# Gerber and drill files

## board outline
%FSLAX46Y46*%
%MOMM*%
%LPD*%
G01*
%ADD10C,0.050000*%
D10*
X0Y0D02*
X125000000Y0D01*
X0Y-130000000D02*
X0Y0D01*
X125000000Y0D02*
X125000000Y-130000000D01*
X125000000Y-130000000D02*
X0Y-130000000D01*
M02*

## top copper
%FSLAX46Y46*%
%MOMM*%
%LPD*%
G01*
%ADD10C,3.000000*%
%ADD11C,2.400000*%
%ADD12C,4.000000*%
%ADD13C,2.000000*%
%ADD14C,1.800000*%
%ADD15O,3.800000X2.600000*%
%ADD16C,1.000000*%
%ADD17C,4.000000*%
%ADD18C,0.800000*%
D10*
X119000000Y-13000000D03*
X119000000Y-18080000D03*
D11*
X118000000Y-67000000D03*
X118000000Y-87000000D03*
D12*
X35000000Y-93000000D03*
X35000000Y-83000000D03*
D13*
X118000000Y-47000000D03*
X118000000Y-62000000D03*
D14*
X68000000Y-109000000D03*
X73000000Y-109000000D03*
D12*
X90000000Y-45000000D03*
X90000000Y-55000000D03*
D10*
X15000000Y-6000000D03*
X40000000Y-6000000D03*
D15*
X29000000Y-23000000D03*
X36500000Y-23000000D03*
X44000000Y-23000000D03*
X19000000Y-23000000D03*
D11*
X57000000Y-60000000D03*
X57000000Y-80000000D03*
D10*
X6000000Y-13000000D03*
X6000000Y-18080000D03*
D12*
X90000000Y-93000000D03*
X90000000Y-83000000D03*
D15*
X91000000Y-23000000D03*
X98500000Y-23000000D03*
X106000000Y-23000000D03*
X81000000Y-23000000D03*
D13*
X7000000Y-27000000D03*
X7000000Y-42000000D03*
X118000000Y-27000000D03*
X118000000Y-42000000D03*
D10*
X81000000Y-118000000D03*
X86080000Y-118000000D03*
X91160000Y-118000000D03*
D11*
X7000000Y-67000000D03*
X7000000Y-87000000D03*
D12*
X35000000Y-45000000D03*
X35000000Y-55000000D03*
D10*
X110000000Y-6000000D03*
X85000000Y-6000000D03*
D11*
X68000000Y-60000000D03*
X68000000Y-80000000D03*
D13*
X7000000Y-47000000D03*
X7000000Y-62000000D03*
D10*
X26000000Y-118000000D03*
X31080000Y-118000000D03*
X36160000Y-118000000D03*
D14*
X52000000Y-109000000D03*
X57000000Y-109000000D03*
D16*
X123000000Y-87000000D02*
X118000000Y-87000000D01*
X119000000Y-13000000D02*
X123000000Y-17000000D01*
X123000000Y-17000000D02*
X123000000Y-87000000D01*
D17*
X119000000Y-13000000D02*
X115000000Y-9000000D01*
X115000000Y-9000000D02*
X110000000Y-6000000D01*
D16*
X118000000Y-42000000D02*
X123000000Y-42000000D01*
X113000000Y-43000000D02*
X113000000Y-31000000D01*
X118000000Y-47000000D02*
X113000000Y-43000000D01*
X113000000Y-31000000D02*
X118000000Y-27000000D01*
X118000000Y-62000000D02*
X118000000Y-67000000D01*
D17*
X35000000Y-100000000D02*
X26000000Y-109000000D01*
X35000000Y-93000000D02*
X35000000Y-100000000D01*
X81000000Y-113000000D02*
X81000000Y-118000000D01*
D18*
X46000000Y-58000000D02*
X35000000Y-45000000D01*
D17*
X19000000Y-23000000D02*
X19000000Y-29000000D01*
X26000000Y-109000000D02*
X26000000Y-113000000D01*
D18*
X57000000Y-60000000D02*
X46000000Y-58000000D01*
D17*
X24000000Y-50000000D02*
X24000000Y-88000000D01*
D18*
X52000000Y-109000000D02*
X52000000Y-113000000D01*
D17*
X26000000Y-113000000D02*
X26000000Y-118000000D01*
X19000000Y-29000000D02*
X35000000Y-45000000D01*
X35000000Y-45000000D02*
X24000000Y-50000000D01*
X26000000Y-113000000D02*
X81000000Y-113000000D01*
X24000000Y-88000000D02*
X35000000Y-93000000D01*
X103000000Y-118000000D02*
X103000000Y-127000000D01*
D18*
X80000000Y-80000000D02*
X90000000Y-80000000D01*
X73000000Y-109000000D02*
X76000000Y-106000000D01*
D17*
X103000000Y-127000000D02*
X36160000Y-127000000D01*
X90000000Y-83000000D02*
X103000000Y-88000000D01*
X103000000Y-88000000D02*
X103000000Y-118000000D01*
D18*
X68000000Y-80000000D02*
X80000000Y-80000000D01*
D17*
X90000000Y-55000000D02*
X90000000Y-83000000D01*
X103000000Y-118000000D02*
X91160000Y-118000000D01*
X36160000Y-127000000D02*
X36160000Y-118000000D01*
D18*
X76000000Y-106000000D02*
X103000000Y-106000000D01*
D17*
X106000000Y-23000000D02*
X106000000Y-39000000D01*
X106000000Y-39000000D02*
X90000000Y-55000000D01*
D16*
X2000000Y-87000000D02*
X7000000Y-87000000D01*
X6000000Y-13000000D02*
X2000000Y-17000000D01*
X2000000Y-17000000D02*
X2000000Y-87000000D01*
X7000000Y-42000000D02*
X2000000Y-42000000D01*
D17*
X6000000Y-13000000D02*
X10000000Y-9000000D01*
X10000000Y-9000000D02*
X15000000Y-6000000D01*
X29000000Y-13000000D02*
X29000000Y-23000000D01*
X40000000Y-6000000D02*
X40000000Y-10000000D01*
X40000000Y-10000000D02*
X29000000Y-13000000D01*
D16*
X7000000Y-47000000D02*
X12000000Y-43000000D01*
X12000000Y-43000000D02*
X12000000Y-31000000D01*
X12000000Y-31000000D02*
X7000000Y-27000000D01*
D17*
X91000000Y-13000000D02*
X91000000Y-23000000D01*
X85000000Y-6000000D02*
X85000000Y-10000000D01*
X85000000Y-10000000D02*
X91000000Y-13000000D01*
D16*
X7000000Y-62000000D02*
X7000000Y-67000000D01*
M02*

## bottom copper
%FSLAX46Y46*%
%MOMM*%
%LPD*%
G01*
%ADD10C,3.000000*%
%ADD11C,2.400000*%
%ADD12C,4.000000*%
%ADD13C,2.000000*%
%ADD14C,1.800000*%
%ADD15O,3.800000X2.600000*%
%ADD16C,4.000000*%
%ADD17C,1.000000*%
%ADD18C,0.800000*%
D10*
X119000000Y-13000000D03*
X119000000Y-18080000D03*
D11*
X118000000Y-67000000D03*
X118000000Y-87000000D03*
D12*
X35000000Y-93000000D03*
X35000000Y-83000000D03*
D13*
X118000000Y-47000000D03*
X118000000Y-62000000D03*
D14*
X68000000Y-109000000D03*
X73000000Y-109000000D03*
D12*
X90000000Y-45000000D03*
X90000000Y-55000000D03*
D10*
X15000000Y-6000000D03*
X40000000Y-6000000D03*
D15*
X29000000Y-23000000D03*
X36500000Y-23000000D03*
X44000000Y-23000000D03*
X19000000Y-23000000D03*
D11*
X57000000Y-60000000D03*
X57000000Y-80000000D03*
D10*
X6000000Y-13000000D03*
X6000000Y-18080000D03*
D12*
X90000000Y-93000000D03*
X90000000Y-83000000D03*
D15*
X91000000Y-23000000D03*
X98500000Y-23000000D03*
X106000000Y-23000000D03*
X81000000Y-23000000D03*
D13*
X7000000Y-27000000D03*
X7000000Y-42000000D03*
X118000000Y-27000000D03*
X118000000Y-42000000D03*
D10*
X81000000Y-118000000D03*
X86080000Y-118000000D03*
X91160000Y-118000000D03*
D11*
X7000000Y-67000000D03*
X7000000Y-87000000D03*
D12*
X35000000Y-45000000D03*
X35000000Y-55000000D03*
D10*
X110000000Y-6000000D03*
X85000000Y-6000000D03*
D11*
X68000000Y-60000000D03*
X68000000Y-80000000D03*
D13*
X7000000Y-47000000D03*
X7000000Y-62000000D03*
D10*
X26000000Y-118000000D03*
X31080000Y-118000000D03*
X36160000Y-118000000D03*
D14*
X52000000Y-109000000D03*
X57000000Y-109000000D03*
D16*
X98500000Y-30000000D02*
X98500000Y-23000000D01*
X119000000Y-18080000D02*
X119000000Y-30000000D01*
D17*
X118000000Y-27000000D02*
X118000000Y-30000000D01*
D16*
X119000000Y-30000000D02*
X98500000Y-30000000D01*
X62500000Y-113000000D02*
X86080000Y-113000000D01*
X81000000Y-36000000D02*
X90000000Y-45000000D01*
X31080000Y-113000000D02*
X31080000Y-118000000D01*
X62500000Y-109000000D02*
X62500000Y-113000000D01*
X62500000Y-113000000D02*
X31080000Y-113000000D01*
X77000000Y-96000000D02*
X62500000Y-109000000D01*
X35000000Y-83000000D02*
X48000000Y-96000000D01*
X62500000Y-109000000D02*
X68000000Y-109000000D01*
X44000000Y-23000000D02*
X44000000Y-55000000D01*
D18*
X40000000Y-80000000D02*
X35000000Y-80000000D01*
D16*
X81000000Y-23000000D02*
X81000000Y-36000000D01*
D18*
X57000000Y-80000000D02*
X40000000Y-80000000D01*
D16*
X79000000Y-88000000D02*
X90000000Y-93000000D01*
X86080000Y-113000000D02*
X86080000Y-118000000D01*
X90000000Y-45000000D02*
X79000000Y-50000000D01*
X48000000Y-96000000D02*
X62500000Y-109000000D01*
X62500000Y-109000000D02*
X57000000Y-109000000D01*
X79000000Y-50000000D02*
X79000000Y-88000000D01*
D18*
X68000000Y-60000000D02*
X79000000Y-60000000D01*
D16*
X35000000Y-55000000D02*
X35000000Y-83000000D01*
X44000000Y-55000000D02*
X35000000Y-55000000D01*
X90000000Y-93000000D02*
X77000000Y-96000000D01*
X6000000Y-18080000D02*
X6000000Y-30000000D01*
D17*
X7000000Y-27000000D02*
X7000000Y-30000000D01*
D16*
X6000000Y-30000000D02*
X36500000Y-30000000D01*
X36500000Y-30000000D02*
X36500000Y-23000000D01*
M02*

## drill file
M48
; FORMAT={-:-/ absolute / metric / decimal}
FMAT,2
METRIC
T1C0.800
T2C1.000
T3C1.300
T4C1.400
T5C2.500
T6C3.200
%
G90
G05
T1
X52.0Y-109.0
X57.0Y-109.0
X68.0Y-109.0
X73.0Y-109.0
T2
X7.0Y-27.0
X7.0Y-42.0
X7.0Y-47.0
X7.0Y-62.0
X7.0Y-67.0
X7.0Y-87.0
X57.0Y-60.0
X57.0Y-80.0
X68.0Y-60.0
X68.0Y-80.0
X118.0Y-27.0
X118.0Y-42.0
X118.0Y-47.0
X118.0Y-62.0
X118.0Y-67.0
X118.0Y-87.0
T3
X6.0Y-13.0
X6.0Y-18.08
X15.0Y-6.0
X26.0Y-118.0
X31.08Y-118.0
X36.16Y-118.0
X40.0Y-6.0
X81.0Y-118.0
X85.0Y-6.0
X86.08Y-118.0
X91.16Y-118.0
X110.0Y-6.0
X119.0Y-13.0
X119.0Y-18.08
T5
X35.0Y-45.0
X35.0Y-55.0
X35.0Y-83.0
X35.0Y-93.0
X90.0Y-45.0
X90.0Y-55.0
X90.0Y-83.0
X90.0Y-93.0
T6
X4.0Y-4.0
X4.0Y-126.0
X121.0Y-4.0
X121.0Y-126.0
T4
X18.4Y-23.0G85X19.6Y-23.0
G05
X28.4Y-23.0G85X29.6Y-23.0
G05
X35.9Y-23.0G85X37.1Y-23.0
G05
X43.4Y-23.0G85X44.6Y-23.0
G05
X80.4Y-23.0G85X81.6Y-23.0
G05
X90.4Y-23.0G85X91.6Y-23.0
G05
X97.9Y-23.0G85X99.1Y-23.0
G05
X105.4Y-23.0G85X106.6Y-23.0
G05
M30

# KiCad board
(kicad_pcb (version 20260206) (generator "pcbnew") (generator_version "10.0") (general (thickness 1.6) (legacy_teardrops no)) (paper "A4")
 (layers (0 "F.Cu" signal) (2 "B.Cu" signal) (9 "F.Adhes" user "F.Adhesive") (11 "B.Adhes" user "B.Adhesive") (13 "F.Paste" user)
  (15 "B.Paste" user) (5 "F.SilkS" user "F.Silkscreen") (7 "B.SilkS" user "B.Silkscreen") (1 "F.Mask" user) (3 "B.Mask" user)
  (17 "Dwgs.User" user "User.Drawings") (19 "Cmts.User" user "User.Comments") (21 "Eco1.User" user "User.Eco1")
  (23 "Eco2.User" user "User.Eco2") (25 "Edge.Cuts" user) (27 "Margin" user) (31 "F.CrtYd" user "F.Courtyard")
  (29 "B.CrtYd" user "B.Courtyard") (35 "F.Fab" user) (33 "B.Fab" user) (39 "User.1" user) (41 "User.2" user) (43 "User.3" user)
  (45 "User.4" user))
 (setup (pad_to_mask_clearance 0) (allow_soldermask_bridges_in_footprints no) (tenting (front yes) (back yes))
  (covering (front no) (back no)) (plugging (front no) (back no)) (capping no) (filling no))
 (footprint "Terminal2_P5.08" (layer "F.Cu") (at 119 13 -90)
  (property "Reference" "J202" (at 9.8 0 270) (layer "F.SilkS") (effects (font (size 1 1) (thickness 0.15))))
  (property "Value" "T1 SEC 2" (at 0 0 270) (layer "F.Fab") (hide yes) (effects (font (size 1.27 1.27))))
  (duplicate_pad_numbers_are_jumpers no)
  (pad "1" thru_hole circle (at 0 0 270) (size 3 3) (drill 1.3) (layers "*.Cu" "*.Mask") (remove_unused_layers no) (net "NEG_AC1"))
  (pad "2" thru_hole circle (at 5.08 0 270) (size 3 3) (drill 1.3) (layers "*.Cu" "*.Mask") (remove_unused_layers no) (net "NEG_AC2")))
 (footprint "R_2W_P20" (layer "F.Cu") (at 118 67 -90)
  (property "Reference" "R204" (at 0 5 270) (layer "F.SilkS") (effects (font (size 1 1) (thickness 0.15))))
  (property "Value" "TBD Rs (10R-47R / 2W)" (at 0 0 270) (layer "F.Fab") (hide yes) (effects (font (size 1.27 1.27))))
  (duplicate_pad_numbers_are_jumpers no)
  (pad "1" thru_hole circle (at 0 0 270) (size 2.4 2.4) (drill 1) (layers "*.Cu" "*.Mask") (remove_unused_layers no) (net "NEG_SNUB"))
  (pad "2" thru_hole circle (at 20 0 270) (size 2.4 2.4) (drill 1) (layers "*.Cu" "*.Mask") (remove_unused_layers no) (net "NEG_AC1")))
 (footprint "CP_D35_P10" (layer "F.Cu") (at 35 93 90)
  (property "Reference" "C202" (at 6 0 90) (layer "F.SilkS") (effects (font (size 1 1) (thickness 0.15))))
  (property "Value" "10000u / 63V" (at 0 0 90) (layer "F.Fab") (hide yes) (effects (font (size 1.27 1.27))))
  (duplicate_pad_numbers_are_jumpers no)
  (pad "1" thru_hole circle (at 0 0 90) (size 4 4) (drill 2.5) (layers "*.Cu" "*.Mask") (remove_unused_layers no) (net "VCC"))
  (pad "2" thru_hole circle (at 10 0 90) (size 4 4) (drill 2.5) (layers "*.Cu" "*.Mask") (remove_unused_layers no) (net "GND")))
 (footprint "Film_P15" (layer "F.Cu") (at 118 47 -90)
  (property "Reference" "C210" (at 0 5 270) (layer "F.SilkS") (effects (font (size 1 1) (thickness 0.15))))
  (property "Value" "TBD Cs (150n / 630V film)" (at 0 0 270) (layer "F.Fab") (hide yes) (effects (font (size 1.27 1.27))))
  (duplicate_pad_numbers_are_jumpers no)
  (pad "1" thru_hole circle (at 0 0 270) (size 2 2) (drill 1) (layers "*.Cu" "*.Mask") (remove_unused_layers no) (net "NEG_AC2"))
  (pad "2" thru_hole circle (at 15 0 270) (size 2 2) (drill 1) (layers "*.Cu" "*.Mask") (remove_unused_layers no) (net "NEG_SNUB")))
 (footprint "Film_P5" (layer "F.Cu") (at 68 109)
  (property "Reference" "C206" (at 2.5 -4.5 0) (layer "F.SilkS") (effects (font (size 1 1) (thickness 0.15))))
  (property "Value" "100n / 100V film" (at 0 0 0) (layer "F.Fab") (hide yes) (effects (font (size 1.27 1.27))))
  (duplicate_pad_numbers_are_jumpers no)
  (pad "1" thru_hole circle (at 0 0) (size 1.8 1.8) (drill 0.8) (layers "*.Cu" "*.Mask") (remove_unused_layers no) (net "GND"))
  (pad "2" thru_hole circle (at 5 0) (size 1.8 1.8) (drill 0.8) (layers "*.Cu" "*.Mask") (remove_unused_layers no) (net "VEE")))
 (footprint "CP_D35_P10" (layer "F.Cu") (at 90 45 -90)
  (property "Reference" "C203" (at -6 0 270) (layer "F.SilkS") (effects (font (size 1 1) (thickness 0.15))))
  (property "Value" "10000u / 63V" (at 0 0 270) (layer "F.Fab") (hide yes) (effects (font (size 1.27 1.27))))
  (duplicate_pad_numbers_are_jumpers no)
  (pad "1" thru_hole circle (at 0 0 270) (size 4 4) (drill 2.5) (layers "*.Cu" "*.Mask") (remove_unused_layers no) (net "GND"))
  (pad "2" thru_hole circle (at 10 0 270) (size 4 4) (drill 2.5) (layers "*.Cu" "*.Mask") (remove_unused_layers no) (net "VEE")))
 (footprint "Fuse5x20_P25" (layer "F.Cu") (at 15 6)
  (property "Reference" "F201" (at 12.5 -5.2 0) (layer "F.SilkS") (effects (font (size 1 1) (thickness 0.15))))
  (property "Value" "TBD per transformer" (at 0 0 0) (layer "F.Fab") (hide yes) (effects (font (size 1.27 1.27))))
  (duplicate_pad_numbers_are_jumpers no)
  (pad "1" thru_hole circle (at 0 0) (size 3 3) (drill 1.3) (layers "*.Cu" "*.Mask") (remove_unused_layers no) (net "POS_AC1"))
  (pad "2" thru_hole circle (at 25 0) (size 3 3) (drill 1.3) (layers "*.Cu" "*.Mask") (remove_unused_layers no) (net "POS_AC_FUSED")))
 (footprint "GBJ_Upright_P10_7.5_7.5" (layer "F.Cu") (at 19 23)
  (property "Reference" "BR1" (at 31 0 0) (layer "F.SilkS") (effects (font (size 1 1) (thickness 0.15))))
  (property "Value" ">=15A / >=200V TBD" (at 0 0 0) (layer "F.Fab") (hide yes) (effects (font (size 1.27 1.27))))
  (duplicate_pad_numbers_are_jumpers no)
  (pad "AC1" thru_hole oval (at 10 0) (size 3.8 2.6) (drill oval 2.6 1.4) (layers "*.Cu" "*.Mask") (remove_unused_layers no)
   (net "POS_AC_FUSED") (thermal_bridge_angle 45))
  (pad "AC2" thru_hole oval (at 17.5 0) (size 3.8 2.6) (drill oval 2.6 1.4) (layers "*.Cu" "*.Mask") (remove_unused_layers no)
   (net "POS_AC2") (thermal_bridge_angle 45))
  (pad "N" thru_hole oval (at 25 0) (size 3.8 2.6) (drill oval 2.6 1.4) (layers "*.Cu" "*.Mask") (remove_unused_layers no) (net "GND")
   (thermal_bridge_angle 45))
  (pad "P" thru_hole oval (at 0 0) (size 3.8 2.6) (drill oval 2.6 1.4) (layers "*.Cu" "*.Mask") (remove_unused_layers no) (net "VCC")
   (thermal_bridge_angle 45)))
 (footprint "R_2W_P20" (layer "F.Cu") (at 57 60 -90)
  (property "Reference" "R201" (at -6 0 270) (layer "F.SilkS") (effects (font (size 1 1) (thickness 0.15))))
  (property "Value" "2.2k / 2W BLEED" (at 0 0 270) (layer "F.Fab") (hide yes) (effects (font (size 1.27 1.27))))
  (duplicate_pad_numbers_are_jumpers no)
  (pad "1" thru_hole circle (at 0 0 270) (size 2.4 2.4) (drill 1) (layers "*.Cu" "*.Mask") (remove_unused_layers no) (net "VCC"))
  (pad "2" thru_hole circle (at 20 0 270) (size 2.4 2.4) (drill 1) (layers "*.Cu" "*.Mask") (remove_unused_layers no) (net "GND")))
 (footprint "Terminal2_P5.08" (layer "F.Cu") (at 6 13 -90)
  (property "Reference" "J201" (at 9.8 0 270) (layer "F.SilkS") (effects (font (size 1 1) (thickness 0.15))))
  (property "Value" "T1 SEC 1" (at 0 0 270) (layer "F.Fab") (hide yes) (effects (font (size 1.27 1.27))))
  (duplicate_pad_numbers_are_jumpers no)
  (pad "1" thru_hole circle (at 0 0 270) (size 3 3) (drill 1.3) (layers "*.Cu" "*.Mask") (remove_unused_layers no) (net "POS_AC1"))
  (pad "2" thru_hole circle (at 5.08 0 270) (size 3 3) (drill 1.3) (layers "*.Cu" "*.Mask") (remove_unused_layers no) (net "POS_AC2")))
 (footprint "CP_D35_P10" (layer "F.Cu") (at 90 93 90)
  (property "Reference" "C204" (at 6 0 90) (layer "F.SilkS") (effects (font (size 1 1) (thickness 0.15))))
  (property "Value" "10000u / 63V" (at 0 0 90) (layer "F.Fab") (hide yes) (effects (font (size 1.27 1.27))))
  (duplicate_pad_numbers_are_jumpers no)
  (pad "1" thru_hole circle (at 0 0 90) (size 4 4) (drill 2.5) (layers "*.Cu" "*.Mask") (remove_unused_layers no) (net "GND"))
  (pad "2" thru_hole circle (at 10 0 90) (size 4 4) (drill 2.5) (layers "*.Cu" "*.Mask") (remove_unused_layers no) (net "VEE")))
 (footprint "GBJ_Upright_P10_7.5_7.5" (layer "F.Cu") (at 81 23)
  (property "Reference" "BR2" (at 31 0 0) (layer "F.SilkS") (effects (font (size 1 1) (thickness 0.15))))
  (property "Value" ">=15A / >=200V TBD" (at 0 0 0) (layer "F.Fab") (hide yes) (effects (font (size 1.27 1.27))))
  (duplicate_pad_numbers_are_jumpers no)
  (pad "AC1" thru_hole oval (at 10 0) (size 3.8 2.6) (drill oval 2.6 1.4) (layers "*.Cu" "*.Mask") (remove_unused_layers no)
   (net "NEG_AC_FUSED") (thermal_bridge_angle 45))
  (pad "AC2" thru_hole oval (at 17.5 0) (size 3.8 2.6) (drill oval 2.6 1.4) (layers "*.Cu" "*.Mask") (remove_unused_layers no)
   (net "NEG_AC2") (thermal_bridge_angle 45))
  (pad "N" thru_hole oval (at 25 0) (size 3.8 2.6) (drill oval 2.6 1.4) (layers "*.Cu" "*.Mask") (remove_unused_layers no) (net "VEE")
   (thermal_bridge_angle 45))
  (pad "P" thru_hole oval (at 0 0) (size 3.8 2.6) (drill oval 2.6 1.4) (layers "*.Cu" "*.Mask") (remove_unused_layers no) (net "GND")
   (thermal_bridge_angle 45)))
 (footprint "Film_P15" (layer "F.Cu") (at 7 27 -90)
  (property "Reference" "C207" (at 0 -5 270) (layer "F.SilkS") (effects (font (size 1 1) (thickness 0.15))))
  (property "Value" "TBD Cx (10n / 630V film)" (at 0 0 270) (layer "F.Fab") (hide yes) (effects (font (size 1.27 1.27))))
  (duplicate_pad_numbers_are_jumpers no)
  (pad "1" thru_hole circle (at 0 0 270) (size 2 2) (drill 1) (layers "*.Cu" "*.Mask") (remove_unused_layers no) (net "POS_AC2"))
  (pad "2" thru_hole circle (at 15 0 270) (size 2 2) (drill 1) (layers "*.Cu" "*.Mask") (remove_unused_layers no) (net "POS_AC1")))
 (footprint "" (layer "F.Cu") (at 4 4)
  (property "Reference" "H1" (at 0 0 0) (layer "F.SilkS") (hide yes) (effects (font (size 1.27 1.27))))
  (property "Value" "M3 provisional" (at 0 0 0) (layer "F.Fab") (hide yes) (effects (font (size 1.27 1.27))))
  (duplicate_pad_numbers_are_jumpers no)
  (pad "" np_thru_hole circle (at 0 0) (size 3.2 3.2) (drill 3.2) (layers "*.Cu" "*.Mask")))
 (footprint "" (layer "F.Cu") (at 4 126)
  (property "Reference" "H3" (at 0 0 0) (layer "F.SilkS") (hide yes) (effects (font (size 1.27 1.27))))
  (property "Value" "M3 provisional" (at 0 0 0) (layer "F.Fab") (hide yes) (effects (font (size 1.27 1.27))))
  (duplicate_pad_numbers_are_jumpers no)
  (pad "" np_thru_hole circle (at 0 0) (size 3.2 3.2) (drill 3.2) (layers "*.Cu" "*.Mask")))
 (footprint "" (layer "F.Cu") (at 121 126)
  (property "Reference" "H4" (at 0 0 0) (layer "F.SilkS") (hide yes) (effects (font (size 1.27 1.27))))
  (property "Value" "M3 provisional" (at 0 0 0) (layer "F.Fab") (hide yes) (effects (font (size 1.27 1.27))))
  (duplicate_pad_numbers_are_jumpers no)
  (pad "" np_thru_hole circle (at 0 0) (size 3.2 3.2) (drill 3.2) (layers "*.Cu" "*.Mask")))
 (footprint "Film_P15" (layer "F.Cu") (at 118 27 -90)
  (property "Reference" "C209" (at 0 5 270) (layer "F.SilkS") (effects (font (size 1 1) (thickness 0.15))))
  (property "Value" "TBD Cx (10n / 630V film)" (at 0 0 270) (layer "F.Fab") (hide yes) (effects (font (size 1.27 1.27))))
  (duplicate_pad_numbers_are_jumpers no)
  (pad "1" thru_hole circle (at 0 0 270) (size 2 2) (drill 1) (layers "*.Cu" "*.Mask") (remove_unused_layers no) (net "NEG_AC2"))
  (pad "2" thru_hole circle (at 15 0 270) (size 2 2) (drill 1) (layers "*.Cu" "*.Mask") (remove_unused_layers no) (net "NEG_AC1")))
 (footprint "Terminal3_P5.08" (layer "F.Cu") (at 81 118)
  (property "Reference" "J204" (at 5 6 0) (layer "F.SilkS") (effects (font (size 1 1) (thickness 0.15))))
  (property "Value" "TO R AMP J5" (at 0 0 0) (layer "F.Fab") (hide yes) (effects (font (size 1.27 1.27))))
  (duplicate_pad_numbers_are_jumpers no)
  (pad "1" thru_hole circle (at 0 0) (size 3 3) (drill 1.3) (layers "*.Cu" "*.Mask") (remove_unused_layers no) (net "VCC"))
  (pad "2" thru_hole circle (at 5.08 0) (size 3 3) (drill 1.3) (layers "*.Cu" "*.Mask") (remove_unused_layers no) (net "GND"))
  (pad "3" thru_hole circle (at 10.16 0) (size 3 3) (drill 1.3) (layers "*.Cu" "*.Mask") (remove_unused_layers no) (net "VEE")))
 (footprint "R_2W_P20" (layer "F.Cu") (at 7 67 -90)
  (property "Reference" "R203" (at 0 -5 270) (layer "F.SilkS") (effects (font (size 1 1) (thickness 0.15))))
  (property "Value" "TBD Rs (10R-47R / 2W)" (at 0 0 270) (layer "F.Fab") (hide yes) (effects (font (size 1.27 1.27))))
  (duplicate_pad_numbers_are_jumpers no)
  (pad "1" thru_hole circle (at 0 0 270) (size 2.4 2.4) (drill 1) (layers "*.Cu" "*.Mask") (remove_unused_layers no) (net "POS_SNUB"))
  (pad "2" thru_hole circle (at 20 0 270) (size 2.4 2.4) (drill 1) (layers "*.Cu" "*.Mask") (remove_unused_layers no) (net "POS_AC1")))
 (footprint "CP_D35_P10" (layer "F.Cu") (at 35 45 -90)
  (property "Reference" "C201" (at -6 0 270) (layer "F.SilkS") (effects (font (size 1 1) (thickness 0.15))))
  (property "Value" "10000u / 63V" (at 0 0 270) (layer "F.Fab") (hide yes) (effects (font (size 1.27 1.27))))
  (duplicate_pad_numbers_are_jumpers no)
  (pad "1" thru_hole circle (at 0 0 270) (size 4 4) (drill 2.5) (layers "*.Cu" "*.Mask") (remove_unused_layers no) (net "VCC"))
  (pad "2" thru_hole circle (at 10 0 270) (size 4 4) (drill 2.5) (layers "*.Cu" "*.Mask") (remove_unused_layers no) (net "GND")))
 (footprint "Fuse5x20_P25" (layer "F.Cu") (at 110 6 180)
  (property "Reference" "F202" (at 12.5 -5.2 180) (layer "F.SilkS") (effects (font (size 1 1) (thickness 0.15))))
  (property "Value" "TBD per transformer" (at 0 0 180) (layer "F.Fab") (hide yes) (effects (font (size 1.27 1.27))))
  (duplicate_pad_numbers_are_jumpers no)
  (pad "1" thru_hole circle (at 0 0 180) (size 3 3) (drill 1.3) (layers "*.Cu" "*.Mask") (remove_unused_layers no) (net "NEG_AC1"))
  (pad "2" thru_hole circle (at 25 0 180) (size 3 3) (drill 1.3) (layers "*.Cu" "*.Mask") (remove_unused_layers no) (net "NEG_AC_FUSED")))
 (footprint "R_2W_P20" (layer "F.Cu") (at 68 60 -90)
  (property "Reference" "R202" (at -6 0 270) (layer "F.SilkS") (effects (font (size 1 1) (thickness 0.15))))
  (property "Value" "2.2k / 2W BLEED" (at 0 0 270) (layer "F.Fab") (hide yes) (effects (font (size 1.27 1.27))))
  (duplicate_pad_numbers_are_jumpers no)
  (pad "1" thru_hole circle (at 0 0 270) (size 2.4 2.4) (drill 1) (layers "*.Cu" "*.Mask") (remove_unused_layers no) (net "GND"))
  (pad "2" thru_hole circle (at 20 0 270) (size 2.4 2.4) (drill 1) (layers "*.Cu" "*.Mask") (remove_unused_layers no) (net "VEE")))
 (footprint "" (layer "F.Cu") (at 121 4)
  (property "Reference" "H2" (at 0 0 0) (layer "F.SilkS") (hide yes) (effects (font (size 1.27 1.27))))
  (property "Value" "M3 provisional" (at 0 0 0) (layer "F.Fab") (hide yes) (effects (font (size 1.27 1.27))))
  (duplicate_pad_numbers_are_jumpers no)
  (pad "" np_thru_hole circle (at 0 0) (size 3.2 3.2) (drill 3.2) (layers "*.Cu" "*.Mask")))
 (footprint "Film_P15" (layer "F.Cu") (at 7 47 -90)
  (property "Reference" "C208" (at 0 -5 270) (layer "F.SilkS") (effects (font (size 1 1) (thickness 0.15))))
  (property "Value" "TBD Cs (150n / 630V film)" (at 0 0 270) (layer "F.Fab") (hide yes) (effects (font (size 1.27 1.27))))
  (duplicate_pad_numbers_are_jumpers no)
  (pad "1" thru_hole circle (at 0 0 270) (size 2 2) (drill 1) (layers "*.Cu" "*.Mask") (remove_unused_layers no) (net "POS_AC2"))
  (pad "2" thru_hole circle (at 15 0 270) (size 2 2) (drill 1) (layers "*.Cu" "*.Mask") (remove_unused_layers no) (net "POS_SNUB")))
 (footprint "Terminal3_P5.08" (layer "F.Cu") (at 26 118)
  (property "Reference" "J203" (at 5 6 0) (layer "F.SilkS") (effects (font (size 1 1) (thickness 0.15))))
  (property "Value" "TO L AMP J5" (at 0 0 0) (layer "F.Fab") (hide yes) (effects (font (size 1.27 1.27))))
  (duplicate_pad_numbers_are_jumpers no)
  (pad "1" thru_hole circle (at 0 0) (size 3 3) (drill 1.3) (layers "*.Cu" "*.Mask") (remove_unused_layers no) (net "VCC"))
  (pad "2" thru_hole circle (at 5.08 0) (size 3 3) (drill 1.3) (layers "*.Cu" "*.Mask") (remove_unused_layers no) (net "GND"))
  (pad "3" thru_hole circle (at 10.16 0) (size 3 3) (drill 1.3) (layers "*.Cu" "*.Mask") (remove_unused_layers no) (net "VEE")))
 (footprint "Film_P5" (layer "F.Cu") (at 52 109)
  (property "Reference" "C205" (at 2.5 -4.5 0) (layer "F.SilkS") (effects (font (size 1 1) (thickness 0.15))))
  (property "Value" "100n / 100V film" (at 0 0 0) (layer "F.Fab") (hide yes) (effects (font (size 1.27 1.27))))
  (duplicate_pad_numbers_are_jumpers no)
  (pad "1" thru_hole circle (at 0 0) (size 1.8 1.8) (drill 0.8) (layers "*.Cu" "*.Mask") (remove_unused_layers no) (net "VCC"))
  (pad "2" thru_hole circle (at 5 0) (size 1.8 1.8) (drill 0.8) (layers "*.Cu" "*.Mask") (remove_unused_layers no) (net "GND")))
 (gr_line (start 0 0) (end 125 0) (stroke (width 0.05) (type default)) (layer "Edge.Cuts"))
 (gr_line (start 0 130) (end 0 0) (stroke (width 0.05) (type default)) (layer "Edge.Cuts"))
 (gr_line (start 125 0) (end 125 130) (stroke (width 0.05) (type default)) (layer "Edge.Cuts"))
 (gr_line (start 125 130) (end 0 130) (stroke (width 0.05) (type default)) (layer "Edge.Cuts"))
 (segment (start 123 87) (end 118 87) (width 1) (layer "F.Cu") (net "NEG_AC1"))
 (segment (start 119 13) (end 123 17) (width 1) (layer "F.Cu") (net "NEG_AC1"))
 (segment (start 123 17) (end 123 87) (width 1) (layer "F.Cu") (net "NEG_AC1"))
 (segment (start 119 13) (end 115 9) (width 4) (layer "F.Cu") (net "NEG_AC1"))
 (segment (start 115 9) (end 110 6) (width 4) (layer "F.Cu") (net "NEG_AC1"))
 (segment (start 118 42) (end 123 42) (width 1) (layer "F.Cu") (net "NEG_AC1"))
 (segment (start 113 43) (end 113 31) (width 1) (layer "F.Cu") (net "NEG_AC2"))
 (segment (start 118 47) (end 113 43) (width 1) (layer "F.Cu") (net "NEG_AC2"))
 (segment (start 113 31) (end 118 27) (width 1) (layer "F.Cu") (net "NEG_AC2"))
 (segment (start 98.5 30) (end 98.5 23) (width 4) (layer "B.Cu") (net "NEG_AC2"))
 (segment (start 119 18.08) (end 119 30) (width 4) (layer "B.Cu") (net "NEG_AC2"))
 (segment (start 118 27) (end 118 30) (width 1) (layer "B.Cu") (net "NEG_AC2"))
 (segment (start 119 30) (end 98.5 30) (width 4) (layer "B.Cu") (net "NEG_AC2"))
 (segment (start 118 62) (end 118 67) (width 1) (layer "F.Cu") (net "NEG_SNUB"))
 (segment (start 35 100) (end 26 109) (width 4) (layer "F.Cu") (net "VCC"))
 (segment (start 35 93) (end 35 100) (width 4) (layer "F.Cu") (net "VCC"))
 (segment (start 81 113) (end 81 118) (width 4) (layer "F.Cu") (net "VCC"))
 (segment (start 46 58) (end 35 45) (width 0.8) (layer "F.Cu") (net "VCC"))
 (segment (start 19 23) (end 19 29) (width 4) (layer "F.Cu") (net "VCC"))
 (segment (start 26 109) (end 26 113) (width 4) (layer "F.Cu") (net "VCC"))
 (segment (start 57 60) (end 46 58) (width 0.8) (layer "F.Cu") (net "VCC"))
 (segment (start 24 50) (end 24 88) (width 4) (layer "F.Cu") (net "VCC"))
 (segment (start 52 109) (end 52 113) (width 0.8) (layer "F.Cu") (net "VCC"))
 (segment (start 26 113) (end 26 118) (width 4) (layer "F.Cu") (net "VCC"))
 (segment (start 19 29) (end 35 45) (width 4) (layer "F.Cu") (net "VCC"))
 (segment (start 35 45) (end 24 50) (width 4) (layer "F.Cu") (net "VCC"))
 (segment (start 26 113) (end 81 113) (width 4) (layer "F.Cu") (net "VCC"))
 (segment (start 24 88) (end 35 93) (width 4) (layer "F.Cu") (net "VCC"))
 (segment (start 62.5 113) (end 86.08 113) (width 4) (layer "B.Cu") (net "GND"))
 (segment (start 81 36) (end 90 45) (width 4) (layer "B.Cu") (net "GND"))
 (segment (start 31.08 113) (end 31.08 118) (width 4) (layer "B.Cu") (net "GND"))
 (segment (start 62.5 109) (end 62.5 113) (width 4) (layer "B.Cu") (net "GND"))
 (segment (start 62.5 113) (end 31.08 113) (width 4) (layer "B.Cu") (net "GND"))
 (segment (start 77 96) (end 62.5 109) (width 4) (layer "B.Cu") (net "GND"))
 (segment (start 35 83) (end 48 96) (width 4) (layer "B.Cu") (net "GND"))
 (segment (start 62.5 109) (end 68 109) (width 4) (layer "B.Cu") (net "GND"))
 (segment (start 44 23) (end 44 55) (width 4) (layer "B.Cu") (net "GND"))
 (segment (start 40 80) (end 35 80) (width 0.8) (layer "B.Cu") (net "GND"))
 (segment (start 81 23) (end 81 36) (width 4) (layer "B.Cu") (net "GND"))
 (segment (start 57 80) (end 40 80) (width 0.8) (layer "B.Cu") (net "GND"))
 (segment (start 79 88) (end 90 93) (width 4) (layer "B.Cu") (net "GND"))
 (segment (start 86.08 113) (end 86.08 118) (width 4) (layer "B.Cu") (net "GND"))
 (segment (start 90 45) (end 79 50) (width 4) (layer "B.Cu") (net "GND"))
 (segment (start 48 96) (end 62.5 109) (width 4) (layer "B.Cu") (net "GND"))
 (segment (start 62.5 109) (end 57 109) (width 4) (layer "B.Cu") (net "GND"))
 (segment (start 79 50) (end 79 88) (width 4) (layer "B.Cu") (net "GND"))
 (segment (start 68 60) (end 79 60) (width 0.8) (layer "B.Cu") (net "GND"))
 (segment (start 35 55) (end 35 83) (width 4) (layer "B.Cu") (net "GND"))
 (segment (start 44 55) (end 35 55) (width 4) (layer "B.Cu") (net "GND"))
 (segment (start 90 93) (end 77 96) (width 4) (layer "B.Cu") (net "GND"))
 (segment (start 103 118) (end 103 127) (width 4) (layer "F.Cu") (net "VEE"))
 (segment (start 80 80) (end 90 80) (width 0.8) (layer "F.Cu") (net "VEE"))
 (segment (start 73 109) (end 76 106) (width 0.8) (layer "F.Cu") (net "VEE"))
 (segment (start 103 127) (end 36.16 127) (width 4) (layer "F.Cu") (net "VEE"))
 (segment (start 90 83) (end 103 88) (width 4) (layer "F.Cu") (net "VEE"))
 (segment (start 103 88) (end 103 118) (width 4) (layer "F.Cu") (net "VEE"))
 (segment (start 68 80) (end 80 80) (width 0.8) (layer "F.Cu") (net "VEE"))
 (segment (start 90 55) (end 90 83) (width 4) (layer "F.Cu") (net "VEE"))
 (segment (start 103 118) (end 91.16 118) (width 4) (layer "F.Cu") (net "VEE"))
 (segment (start 36.16 127) (end 36.16 118) (width 4) (layer "F.Cu") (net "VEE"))
 (segment (start 76 106) (end 103 106) (width 0.8) (layer "F.Cu") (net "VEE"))
 (segment (start 106 23) (end 106 39) (width 4) (layer "F.Cu") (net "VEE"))
 (segment (start 106 39) (end 90 55) (width 4) (layer "F.Cu") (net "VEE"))
 (segment (start 2 87) (end 7 87) (width 1) (layer "F.Cu") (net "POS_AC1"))
 (segment (start 6 13) (end 2 17) (width 1) (layer "F.Cu") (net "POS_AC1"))
 (segment (start 2 17) (end 2 87) (width 1) (layer "F.Cu") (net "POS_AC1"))
 (segment (start 7 42) (end 2 42) (width 1) (layer "F.Cu") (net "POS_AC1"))
 (segment (start 6 13) (end 10 9) (width 4) (layer "F.Cu") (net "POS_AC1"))
 (segment (start 10 9) (end 15 6) (width 4) (layer "F.Cu") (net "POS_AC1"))
 (segment (start 29 13) (end 29 23) (width 4) (layer "F.Cu") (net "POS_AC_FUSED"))
 (segment (start 40 6) (end 40 10) (width 4) (layer "F.Cu") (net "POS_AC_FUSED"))
 (segment (start 40 10) (end 29 13) (width 4) (layer "F.Cu") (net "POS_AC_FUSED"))
 (segment (start 7 47) (end 12 43) (width 1) (layer "F.Cu") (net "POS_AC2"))
 (segment (start 12 43) (end 12 31) (width 1) (layer "F.Cu") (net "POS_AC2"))
 (segment (start 12 31) (end 7 27) (width 1) (layer "F.Cu") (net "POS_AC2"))
 (segment (start 6 18.08) (end 6 30) (width 4) (layer "B.Cu") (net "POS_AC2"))
 (segment (start 7 27) (end 7 30) (width 1) (layer "B.Cu") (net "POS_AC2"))
 (segment (start 6 30) (end 36.5 30) (width 4) (layer "B.Cu") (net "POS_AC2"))
 (segment (start 36.5 30) (end 36.5 23) (width 4) (layer "B.Cu") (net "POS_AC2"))
 (segment (start 91 13) (end 91 23) (width 4) (layer "F.Cu") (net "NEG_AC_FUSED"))
 (segment (start 85 6) (end 85 10) (width 4) (layer "F.Cu") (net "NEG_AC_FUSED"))
 (segment (start 85 10) (end 91 13) (width 4) (layer "F.Cu") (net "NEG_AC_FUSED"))
 (segment (start 7 62) (end 7 67) (width 1) (layer "F.Cu") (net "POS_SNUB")))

